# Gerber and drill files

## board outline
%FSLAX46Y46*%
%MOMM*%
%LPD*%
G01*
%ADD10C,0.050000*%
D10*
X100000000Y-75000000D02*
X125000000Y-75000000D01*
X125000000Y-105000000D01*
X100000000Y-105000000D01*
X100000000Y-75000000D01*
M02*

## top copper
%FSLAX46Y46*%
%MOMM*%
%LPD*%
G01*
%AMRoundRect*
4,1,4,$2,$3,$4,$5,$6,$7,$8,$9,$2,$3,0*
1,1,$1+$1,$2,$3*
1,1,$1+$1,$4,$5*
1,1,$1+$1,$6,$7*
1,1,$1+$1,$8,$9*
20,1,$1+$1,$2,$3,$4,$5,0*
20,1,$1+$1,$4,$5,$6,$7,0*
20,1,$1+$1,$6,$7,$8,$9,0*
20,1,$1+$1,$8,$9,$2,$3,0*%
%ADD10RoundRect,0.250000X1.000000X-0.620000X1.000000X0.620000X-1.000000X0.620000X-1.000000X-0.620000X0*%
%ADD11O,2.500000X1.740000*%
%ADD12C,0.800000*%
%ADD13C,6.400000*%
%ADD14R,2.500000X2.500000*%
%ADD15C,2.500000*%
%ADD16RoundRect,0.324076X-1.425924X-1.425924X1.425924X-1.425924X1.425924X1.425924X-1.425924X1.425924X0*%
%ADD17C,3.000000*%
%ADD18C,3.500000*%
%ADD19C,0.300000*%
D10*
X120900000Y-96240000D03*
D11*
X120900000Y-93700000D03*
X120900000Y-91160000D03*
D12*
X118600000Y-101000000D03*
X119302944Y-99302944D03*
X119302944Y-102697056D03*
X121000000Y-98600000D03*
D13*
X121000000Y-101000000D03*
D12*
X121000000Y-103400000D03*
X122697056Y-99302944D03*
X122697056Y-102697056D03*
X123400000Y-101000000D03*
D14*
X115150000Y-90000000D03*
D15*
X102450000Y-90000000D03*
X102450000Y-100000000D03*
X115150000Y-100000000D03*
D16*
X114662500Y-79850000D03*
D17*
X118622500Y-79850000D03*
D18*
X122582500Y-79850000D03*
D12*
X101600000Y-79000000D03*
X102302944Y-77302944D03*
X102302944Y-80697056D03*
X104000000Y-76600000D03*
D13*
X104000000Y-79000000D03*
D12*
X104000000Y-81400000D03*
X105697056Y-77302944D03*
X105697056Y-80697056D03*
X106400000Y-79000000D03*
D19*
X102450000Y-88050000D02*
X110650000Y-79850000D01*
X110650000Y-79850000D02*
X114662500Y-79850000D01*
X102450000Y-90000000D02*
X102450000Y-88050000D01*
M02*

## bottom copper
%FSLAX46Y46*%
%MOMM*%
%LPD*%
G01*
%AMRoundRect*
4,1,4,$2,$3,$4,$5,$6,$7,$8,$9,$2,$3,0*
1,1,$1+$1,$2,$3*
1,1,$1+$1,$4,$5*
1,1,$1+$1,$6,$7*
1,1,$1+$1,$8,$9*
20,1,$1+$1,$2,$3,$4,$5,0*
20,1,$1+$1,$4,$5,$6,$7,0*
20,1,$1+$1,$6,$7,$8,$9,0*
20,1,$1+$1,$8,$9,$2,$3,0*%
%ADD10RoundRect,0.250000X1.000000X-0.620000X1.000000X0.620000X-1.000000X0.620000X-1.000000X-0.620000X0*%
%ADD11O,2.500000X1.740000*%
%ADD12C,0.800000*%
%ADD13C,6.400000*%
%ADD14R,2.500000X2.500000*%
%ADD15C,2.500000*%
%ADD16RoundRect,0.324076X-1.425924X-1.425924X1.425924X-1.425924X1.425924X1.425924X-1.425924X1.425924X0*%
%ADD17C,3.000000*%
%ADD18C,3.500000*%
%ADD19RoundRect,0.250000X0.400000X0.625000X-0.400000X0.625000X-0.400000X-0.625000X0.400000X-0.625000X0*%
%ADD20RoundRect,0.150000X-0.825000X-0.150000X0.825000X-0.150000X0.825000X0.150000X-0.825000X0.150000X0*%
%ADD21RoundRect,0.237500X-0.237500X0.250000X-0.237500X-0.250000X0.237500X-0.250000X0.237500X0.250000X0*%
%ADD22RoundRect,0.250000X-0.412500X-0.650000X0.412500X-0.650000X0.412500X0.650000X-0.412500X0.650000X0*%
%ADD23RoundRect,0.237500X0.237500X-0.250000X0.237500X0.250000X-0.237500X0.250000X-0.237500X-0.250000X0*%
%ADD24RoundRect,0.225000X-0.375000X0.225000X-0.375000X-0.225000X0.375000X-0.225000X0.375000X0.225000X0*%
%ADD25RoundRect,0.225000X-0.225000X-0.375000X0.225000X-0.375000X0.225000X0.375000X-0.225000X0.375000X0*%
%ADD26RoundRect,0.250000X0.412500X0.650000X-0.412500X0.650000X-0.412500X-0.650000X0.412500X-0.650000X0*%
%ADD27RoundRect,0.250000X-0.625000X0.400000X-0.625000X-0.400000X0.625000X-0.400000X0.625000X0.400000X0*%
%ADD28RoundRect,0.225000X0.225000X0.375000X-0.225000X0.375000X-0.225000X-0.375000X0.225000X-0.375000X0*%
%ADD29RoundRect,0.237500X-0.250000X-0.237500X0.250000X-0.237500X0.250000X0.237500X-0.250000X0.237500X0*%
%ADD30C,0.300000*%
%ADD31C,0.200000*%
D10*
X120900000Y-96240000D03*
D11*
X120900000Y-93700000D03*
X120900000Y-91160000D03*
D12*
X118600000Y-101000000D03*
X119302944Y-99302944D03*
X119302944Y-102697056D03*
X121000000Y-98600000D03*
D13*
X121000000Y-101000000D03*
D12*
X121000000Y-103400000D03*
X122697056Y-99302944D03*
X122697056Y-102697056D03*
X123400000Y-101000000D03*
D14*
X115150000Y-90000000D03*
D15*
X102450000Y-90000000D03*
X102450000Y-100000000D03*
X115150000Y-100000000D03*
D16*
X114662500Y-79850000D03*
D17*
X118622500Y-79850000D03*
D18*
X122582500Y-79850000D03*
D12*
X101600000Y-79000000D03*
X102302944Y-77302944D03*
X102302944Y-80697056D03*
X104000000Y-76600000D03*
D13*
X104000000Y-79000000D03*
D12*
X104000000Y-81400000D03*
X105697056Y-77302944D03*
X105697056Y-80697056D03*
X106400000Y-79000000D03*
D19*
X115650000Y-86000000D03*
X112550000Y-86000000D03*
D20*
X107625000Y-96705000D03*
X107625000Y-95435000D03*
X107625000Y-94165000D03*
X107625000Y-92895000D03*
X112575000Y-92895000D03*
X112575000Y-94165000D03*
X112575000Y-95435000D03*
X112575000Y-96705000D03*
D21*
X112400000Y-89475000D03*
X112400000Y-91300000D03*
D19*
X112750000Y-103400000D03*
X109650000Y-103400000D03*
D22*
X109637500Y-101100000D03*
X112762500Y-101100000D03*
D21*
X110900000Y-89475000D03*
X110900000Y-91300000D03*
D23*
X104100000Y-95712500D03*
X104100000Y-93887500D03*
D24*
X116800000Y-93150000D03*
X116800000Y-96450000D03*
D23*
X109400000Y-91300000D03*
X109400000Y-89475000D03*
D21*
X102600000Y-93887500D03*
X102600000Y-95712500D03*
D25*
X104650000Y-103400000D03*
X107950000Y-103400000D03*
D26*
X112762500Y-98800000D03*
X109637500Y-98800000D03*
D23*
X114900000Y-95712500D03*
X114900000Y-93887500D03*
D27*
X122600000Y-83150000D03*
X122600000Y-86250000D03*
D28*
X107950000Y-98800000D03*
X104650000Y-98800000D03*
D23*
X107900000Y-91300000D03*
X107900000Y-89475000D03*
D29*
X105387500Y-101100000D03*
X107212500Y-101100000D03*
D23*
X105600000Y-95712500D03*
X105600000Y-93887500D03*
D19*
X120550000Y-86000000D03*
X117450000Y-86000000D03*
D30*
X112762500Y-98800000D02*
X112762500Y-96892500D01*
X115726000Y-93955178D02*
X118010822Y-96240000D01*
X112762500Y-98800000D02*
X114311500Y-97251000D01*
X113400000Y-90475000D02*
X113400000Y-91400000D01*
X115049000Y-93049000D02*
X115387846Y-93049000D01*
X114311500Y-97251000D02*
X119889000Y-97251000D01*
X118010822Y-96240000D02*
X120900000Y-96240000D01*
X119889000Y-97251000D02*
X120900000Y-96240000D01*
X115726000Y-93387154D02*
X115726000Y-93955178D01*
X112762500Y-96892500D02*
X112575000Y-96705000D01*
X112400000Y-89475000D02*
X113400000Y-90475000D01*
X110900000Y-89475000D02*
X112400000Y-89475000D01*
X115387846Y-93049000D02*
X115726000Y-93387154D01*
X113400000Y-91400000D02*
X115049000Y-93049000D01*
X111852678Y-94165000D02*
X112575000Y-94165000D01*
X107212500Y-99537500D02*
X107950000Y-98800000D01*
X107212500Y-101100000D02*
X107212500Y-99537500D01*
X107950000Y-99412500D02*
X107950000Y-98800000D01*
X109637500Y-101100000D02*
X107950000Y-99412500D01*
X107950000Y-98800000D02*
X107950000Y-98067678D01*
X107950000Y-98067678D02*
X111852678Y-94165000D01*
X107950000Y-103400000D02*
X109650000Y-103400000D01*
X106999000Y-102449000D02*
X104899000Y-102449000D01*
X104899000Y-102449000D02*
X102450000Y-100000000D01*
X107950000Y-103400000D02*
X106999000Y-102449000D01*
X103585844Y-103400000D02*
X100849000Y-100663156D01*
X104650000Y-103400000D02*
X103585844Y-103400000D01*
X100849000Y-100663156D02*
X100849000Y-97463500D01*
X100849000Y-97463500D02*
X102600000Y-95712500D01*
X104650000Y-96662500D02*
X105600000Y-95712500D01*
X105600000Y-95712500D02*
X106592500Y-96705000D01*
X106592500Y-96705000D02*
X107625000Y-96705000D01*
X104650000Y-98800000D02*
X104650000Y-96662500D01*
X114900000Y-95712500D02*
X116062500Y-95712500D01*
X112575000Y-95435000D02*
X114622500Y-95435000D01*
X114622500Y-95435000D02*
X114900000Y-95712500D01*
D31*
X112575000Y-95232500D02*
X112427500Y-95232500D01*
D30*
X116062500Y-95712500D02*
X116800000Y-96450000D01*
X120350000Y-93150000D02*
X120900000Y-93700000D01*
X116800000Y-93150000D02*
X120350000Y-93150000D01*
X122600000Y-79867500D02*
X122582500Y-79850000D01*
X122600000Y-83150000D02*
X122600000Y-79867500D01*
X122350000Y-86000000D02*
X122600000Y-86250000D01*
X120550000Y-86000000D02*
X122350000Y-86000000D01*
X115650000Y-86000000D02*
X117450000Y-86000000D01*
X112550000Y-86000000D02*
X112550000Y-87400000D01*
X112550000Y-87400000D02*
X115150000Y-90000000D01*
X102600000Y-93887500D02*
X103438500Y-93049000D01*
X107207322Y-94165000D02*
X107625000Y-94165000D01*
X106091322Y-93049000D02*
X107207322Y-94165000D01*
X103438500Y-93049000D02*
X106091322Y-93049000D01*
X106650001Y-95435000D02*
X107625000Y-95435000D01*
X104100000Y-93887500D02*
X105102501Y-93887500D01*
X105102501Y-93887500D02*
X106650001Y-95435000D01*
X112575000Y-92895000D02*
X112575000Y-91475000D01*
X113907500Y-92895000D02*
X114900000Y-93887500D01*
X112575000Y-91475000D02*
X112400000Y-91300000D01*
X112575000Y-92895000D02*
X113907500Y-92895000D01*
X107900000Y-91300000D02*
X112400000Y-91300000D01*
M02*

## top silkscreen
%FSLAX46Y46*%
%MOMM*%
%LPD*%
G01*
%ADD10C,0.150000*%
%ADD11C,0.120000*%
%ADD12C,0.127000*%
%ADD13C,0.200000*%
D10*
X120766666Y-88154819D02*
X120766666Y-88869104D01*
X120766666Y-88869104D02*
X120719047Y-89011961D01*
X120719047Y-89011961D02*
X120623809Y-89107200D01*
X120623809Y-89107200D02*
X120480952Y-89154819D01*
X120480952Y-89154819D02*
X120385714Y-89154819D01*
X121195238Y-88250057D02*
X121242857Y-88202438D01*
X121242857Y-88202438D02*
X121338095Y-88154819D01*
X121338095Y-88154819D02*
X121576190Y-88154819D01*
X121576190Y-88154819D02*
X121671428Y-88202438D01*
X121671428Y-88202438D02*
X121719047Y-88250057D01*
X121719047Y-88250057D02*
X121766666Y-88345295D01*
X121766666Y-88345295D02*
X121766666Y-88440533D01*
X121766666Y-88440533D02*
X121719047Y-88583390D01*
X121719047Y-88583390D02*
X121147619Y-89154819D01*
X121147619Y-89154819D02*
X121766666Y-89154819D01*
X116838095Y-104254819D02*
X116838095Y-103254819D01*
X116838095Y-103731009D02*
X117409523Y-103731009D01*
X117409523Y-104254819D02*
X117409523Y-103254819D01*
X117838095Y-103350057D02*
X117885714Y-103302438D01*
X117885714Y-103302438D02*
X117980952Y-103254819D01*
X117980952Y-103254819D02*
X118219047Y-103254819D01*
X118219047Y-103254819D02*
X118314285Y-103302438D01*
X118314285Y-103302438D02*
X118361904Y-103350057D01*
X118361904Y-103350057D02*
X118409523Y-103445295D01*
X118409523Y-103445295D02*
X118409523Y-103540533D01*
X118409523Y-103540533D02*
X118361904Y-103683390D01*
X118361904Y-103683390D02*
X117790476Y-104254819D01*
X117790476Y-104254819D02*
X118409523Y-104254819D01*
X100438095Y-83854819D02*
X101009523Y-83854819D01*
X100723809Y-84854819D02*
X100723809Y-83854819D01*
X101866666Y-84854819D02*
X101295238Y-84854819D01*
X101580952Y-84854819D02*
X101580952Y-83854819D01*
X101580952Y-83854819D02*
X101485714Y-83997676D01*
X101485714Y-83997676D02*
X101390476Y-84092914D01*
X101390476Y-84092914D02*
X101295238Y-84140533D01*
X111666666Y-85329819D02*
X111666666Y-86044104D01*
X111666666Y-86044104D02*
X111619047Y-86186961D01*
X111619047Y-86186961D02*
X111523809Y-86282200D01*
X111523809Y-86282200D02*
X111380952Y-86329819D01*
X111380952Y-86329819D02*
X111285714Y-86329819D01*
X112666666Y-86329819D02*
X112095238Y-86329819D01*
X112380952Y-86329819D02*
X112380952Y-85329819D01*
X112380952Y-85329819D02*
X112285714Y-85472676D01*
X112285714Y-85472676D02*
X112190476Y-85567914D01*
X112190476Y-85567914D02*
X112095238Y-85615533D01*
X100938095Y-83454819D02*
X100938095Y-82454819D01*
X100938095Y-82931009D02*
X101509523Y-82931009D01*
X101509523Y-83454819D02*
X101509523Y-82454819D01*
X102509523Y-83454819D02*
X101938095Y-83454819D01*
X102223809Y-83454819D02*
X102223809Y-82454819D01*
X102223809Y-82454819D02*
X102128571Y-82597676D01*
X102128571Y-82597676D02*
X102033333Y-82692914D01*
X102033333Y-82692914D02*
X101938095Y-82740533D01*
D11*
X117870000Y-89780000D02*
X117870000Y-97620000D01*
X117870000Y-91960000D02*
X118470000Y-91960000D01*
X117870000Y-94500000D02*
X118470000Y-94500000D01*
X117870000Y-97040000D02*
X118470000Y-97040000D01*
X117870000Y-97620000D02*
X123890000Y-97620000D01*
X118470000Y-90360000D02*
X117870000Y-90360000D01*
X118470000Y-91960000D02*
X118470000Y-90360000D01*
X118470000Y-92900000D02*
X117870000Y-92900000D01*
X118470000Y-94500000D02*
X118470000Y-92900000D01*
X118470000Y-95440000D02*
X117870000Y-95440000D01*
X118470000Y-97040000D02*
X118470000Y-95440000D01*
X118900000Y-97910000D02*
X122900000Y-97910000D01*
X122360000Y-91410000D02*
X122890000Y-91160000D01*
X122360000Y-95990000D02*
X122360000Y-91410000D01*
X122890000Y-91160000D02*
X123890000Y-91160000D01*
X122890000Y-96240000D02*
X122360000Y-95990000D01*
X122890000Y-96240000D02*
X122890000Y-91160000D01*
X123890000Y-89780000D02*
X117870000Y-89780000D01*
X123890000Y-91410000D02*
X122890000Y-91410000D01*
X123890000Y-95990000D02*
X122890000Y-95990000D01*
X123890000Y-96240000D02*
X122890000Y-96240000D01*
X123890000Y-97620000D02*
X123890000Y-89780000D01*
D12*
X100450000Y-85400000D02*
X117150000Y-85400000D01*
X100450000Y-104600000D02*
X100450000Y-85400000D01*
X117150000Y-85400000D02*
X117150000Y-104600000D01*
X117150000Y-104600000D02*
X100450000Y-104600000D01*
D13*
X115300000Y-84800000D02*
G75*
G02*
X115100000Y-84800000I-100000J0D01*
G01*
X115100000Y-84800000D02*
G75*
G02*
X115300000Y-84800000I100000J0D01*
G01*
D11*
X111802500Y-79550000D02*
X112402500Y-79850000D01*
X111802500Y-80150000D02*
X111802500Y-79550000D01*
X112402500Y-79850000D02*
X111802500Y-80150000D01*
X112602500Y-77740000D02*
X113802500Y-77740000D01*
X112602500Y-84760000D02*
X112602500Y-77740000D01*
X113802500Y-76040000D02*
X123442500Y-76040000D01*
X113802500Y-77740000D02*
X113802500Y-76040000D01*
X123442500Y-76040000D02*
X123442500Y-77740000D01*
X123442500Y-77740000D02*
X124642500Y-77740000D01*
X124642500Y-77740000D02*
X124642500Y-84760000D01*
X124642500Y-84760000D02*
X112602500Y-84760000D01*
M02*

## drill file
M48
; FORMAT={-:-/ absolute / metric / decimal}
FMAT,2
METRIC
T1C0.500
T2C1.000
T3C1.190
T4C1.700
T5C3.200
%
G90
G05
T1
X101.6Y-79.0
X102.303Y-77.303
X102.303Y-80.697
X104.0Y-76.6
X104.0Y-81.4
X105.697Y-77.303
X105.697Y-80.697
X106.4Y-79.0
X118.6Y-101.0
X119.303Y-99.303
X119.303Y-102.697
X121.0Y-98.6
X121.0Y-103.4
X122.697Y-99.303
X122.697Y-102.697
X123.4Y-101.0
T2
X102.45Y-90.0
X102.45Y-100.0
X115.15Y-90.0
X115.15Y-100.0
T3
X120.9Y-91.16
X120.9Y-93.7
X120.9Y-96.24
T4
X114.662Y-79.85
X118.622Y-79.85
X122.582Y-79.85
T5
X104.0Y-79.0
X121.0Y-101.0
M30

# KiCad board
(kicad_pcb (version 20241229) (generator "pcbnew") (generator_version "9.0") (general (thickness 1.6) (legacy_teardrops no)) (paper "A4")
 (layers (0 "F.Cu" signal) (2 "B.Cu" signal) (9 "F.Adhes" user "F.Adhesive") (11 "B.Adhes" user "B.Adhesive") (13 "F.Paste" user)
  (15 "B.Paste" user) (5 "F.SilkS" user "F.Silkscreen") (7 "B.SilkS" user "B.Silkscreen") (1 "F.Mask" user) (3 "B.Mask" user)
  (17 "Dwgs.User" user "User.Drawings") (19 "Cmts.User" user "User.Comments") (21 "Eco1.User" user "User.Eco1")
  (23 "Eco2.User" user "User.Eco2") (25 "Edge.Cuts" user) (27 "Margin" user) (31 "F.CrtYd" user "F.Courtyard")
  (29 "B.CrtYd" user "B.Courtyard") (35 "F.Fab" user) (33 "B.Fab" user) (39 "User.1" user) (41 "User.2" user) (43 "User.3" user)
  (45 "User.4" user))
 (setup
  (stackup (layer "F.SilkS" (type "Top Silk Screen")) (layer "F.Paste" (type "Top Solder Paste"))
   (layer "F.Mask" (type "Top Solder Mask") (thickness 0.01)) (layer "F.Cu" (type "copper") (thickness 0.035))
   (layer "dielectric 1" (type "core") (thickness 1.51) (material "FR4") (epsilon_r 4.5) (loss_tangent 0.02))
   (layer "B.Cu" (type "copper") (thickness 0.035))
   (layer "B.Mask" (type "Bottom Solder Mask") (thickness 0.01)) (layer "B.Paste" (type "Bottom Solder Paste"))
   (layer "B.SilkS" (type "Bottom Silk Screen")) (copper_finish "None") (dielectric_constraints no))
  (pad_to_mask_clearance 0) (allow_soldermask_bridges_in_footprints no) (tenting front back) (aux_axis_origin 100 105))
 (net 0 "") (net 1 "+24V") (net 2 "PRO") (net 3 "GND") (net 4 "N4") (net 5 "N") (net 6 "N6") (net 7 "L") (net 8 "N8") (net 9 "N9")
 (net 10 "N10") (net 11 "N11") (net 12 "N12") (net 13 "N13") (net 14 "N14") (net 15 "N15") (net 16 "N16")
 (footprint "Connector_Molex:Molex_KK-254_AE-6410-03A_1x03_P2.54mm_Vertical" (layer "F.Cu") (at 120.9 96.24 90)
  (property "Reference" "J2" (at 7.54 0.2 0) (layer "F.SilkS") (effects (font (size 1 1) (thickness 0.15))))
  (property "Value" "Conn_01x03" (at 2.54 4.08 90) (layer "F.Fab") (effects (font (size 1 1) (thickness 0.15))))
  (fp_line (start 6.46 -3.03) (end -1.38 -3.03) (stroke (width 0.12) (type solid)) (layer "F.SilkS"))
  (fp_line (start 4.28 -3.03) (end 4.28 -2.43) (stroke (width 0.12) (type solid)) (layer "F.SilkS"))
  (fp_line (start 1.74 -3.03) (end 1.74 -2.43) (stroke (width 0.12) (type solid)) (layer "F.SilkS"))
  (fp_line (start -0.8 -3.03) (end -0.8 -2.43) (stroke (width 0.12) (type solid)) (layer "F.SilkS"))
  (fp_line (start -1.38 -3.03) (end -1.38 2.99) (stroke (width 0.12) (type solid)) (layer "F.SilkS"))
  (fp_line (start 5.88 -2.43) (end 5.88 -3.03) (stroke (width 0.12) (type solid)) (layer "F.SilkS"))
  (fp_line (start 4.28 -2.43) (end 5.88 -2.43) (stroke (width 0.12) (type solid)) (layer "F.SilkS"))
  (fp_line (start 3.34 -2.43) (end 3.34 -3.03) (stroke (width 0.12) (type solid)) (layer "F.SilkS"))
  (fp_line (start 1.74 -2.43) (end 3.34 -2.43) (stroke (width 0.12) (type solid)) (layer "F.SilkS"))
  (fp_line (start 0.8 -2.43) (end 0.8 -3.03) (stroke (width 0.12) (type solid)) (layer "F.SilkS"))
  (fp_line (start -0.8 -2.43) (end 0.8 -2.43) (stroke (width 0.12) (type solid)) (layer "F.SilkS"))
  (fp_line (start -1.67 -2) (end -1.67 2) (stroke (width 0.12) (type solid)) (layer "F.SilkS"))
  (fp_line (start 4.83 1.46) (end 5.08 1.99) (stroke (width 0.12) (type solid)) (layer "F.SilkS"))
  (fp_line (start 0.25 1.46) (end 4.83 1.46) (stroke (width 0.12) (type solid)) (layer "F.SilkS"))
  (fp_line (start 5.08 1.99) (end 5.08 2.99) (stroke (width 0.12) (type solid)) (layer "F.SilkS"))
  (fp_line (start 0 1.99) (end 0.25 1.46) (stroke (width 0.12) (type solid)) (layer "F.SilkS"))
  (fp_line (start 0 1.99) (end 5.08 1.99) (stroke (width 0.12) (type solid)) (layer "F.SilkS"))
  (fp_line (start 6.46 2.99) (end 6.46 -3.03) (stroke (width 0.12) (type solid)) (layer "F.SilkS"))
  (fp_line (start 4.83 2.99) (end 4.83 1.99) (stroke (width 0.12) (type solid)) (layer "F.SilkS"))
  (fp_line (start 0.25 2.99) (end 0.25 1.99) (stroke (width 0.12) (type solid)) (layer "F.SilkS"))
  (fp_line (start 0 2.99) (end 0 1.99) (stroke (width 0.12) (type solid)) (layer "F.SilkS"))
  (fp_line (start -1.38 2.99) (end 6.46 2.99) (stroke (width 0.12) (type solid)) (layer "F.SilkS"))
  (pad "1" thru_hole roundrect (at 0 0 90) (size 1.74 2.5) (drill 1.19) (layers "*.Cu" "*.Mask") (remove_unused_layers no)
   (roundrect_rratio 0.143678) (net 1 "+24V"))
  (pad "2" thru_hole oval (at 2.54 0 90) (size 1.74 2.5) (drill 1.19) (layers "*.Cu" "*.Mask") (remove_unused_layers no) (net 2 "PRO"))
  (pad "3" thru_hole oval (at 5.08 0 90) (size 1.74 2.5) (drill 1.19) (layers "*.Cu" "*.Mask") (remove_unused_layers no) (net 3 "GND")))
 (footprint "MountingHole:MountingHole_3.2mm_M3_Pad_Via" (layer "F.Cu") (at 121 101)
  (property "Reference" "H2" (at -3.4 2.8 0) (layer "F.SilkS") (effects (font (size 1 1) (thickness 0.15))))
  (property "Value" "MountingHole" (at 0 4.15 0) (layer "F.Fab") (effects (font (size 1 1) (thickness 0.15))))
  (pad "1" thru_hole circle (at -2.4 0) (size 0.8 0.8) (drill 0.5) (layers "*.Cu" "*.Mask") (remove_unused_layers no) (zone_connect 2))
  (pad "1" thru_hole circle (at -1.697056 -1.697056) (size 0.8 0.8) (drill 0.5) (layers "*.Cu" "*.Mask") (remove_unused_layers no)
   (zone_connect 2))
  (pad "1" thru_hole circle (at -1.697056 1.697056) (size 0.8 0.8) (drill 0.5) (layers "*.Cu" "*.Mask") (remove_unused_layers no)
   (zone_connect 2))
  (pad "1" thru_hole circle (at 0 -2.4) (size 0.8 0.8) (drill 0.5) (layers "*.Cu" "*.Mask") (remove_unused_layers no) (zone_connect 2))
  (pad "1" thru_hole circle (at 0 0) (size 6.4 6.4) (drill 3.2) (layers "*.Cu" "*.Mask") (remove_unused_layers no) (zone_connect 2))
  (pad "1" thru_hole circle (at 0 2.4) (size 0.8 0.8) (drill 0.5) (layers "*.Cu" "*.Mask") (remove_unused_layers no) (zone_connect 2))
  (pad "1" thru_hole circle (at 1.697056 -1.697056) (size 0.8 0.8) (drill 0.5) (layers "*.Cu" "*.Mask") (remove_unused_layers no)
   (zone_connect 2))
  (pad "1" thru_hole circle (at 1.697056 1.697056) (size 0.8 0.8) (drill 0.5) (layers "*.Cu" "*.Mask") (remove_unused_layers no)
   (zone_connect 2))
  (pad "1" thru_hole circle (at 2.4 0) (size 0.8 0.8) (drill 0.5) (layers "*.Cu" "*.Mask") (remove_unused_layers no) (zone_connect 2)))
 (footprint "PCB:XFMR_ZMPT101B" (layer "F.Cu") (at 108.8 95 -90)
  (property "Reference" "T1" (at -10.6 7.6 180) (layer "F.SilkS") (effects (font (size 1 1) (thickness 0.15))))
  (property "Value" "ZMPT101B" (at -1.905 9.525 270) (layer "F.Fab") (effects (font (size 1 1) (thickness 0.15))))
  (fp_line (start -9.6 8.35) (end -9.6 -8.35) (stroke (width 0.127) (type solid)) (layer "F.SilkS"))
  (fp_line (start 9.6 8.35) (end -9.6 8.35) (stroke (width 0.127) (type solid)) (layer "F.SilkS"))
  (fp_line (start -9.6 -8.35) (end 9.6 -8.35) (stroke (width 0.127) (type solid)) (layer "F.SilkS"))
  (fp_line (start 9.6 -8.35) (end 9.6 8.35) (stroke (width 0.127) (type solid)) (layer "F.SilkS"))
  (fp_circle (center -10.2 -6.4) (end -10.1 -6.4) (stroke (width 0.2) (type solid)) (fill no) (layer "F.SilkS"))
  (pad "1" thru_hole rect (at -5 -6.35 270) (size 2.5 2.5) (drill 1) (layers "*.Cu" "*.Mask") (remove_unused_layers no) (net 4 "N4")
   (solder_mask_margin 0.102))
  (pad "2" thru_hole circle (at -5 6.35 270) (size 2.5 2.5) (drill 1) (layers "*.Cu" "*.Mask") (remove_unused_layers no) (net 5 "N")
   (solder_mask_margin 0.102))
  (pad "3" thru_hole circle (at 5 6.35 270) (size 2.5 2.5) (drill 1) (layers "*.Cu" "*.Mask") (remove_unused_layers no) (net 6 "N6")
   (solder_mask_margin 0.102))
  (pad "4" thru_hole circle (at 5 -6.35 270) (size 2.5 2.5) (drill 1) (layers "*.Cu" "*.Mask") (remove_unused_layers no) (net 3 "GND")
   (solder_mask_margin 0.102)))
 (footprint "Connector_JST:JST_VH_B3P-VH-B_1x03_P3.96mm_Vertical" (layer "F.Cu") (at 114.6625 79.85)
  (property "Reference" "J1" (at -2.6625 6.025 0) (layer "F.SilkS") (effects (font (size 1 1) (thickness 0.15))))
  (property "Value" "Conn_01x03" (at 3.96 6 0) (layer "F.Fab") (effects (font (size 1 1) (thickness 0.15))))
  (fp_line (start -2.86 -0.3) (end -2.26 0) (stroke (width 0.12) (type solid)) (layer "F.SilkS"))
  (fp_line (start -2.86 0.3) (end -2.86 -0.3) (stroke (width 0.12) (type solid)) (layer "F.SilkS"))
  (fp_line (start -2.26 0) (end -2.86 0.3) (stroke (width 0.12) (type solid)) (layer "F.SilkS"))
  (fp_line (start -2.06 -2.11) (end -0.86 -2.11) (stroke (width 0.12) (type solid)) (layer "F.SilkS"))
  (fp_line (start -2.06 4.91) (end -2.06 -2.11) (stroke (width 0.12) (type solid)) (layer "F.SilkS"))
  (fp_line (start -0.86 -3.81) (end 8.78 -3.81) (stroke (width 0.12) (type solid)) (layer "F.SilkS"))
  (fp_line (start -0.86 -2.11) (end -0.86 -3.81) (stroke (width 0.12) (type solid)) (layer "F.SilkS"))
  (fp_line (start 8.78 -3.81) (end 8.78 -2.11) (stroke (width 0.12) (type solid)) (layer "F.SilkS"))
  (fp_line (start 8.78 -2.11) (end 9.98 -2.11) (stroke (width 0.12) (type solid)) (layer "F.SilkS"))
  (fp_line (start 9.98 -2.11) (end 9.98 4.91) (stroke (width 0.12) (type solid)) (layer "F.SilkS"))
  (fp_line (start 9.98 4.91) (end -2.06 4.91) (stroke (width 0.12) (type solid)) (layer "F.SilkS"))
  (pad "1" thru_hole roundrect (at 0 0) (size 3.5 3.5) (drill 1.7) (layers "*.Cu" "*.Mask") (remove_unused_layers no)
   (roundrect_rratio 0.092593) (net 5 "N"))
  (pad "2" thru_hole circle (at 3.96 0) (size 3 3) (drill 1.7) (layers) (remove_unused_layers no))
  (pad "3" thru_hole circle (at 7.92 0) (size 3.5 3.5) (drill 1.7) (layers "*.Cu" "*.Mask") (remove_unused_layers no) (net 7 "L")))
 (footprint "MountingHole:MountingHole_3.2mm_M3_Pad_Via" (layer "F.Cu") (at 104 79)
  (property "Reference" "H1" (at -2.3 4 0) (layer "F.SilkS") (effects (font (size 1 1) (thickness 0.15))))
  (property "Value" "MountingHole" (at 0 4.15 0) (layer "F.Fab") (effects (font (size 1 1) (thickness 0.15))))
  (pad "1" thru_hole circle (at -2.4 0) (size 0.8 0.8) (drill 0.5) (layers "*.Cu" "*.Mask") (remove_unused_layers no) (zone_connect 2))
  (pad "1" thru_hole circle (at -1.697056 -1.697056) (size 0.8 0.8) (drill 0.5) (layers "*.Cu" "*.Mask") (remove_unused_layers no)
   (zone_connect 2))
  (pad "1" thru_hole circle (at -1.697056 1.697056) (size 0.8 0.8) (drill 0.5) (layers "*.Cu" "*.Mask") (remove_unused_layers no)
   (zone_connect 2))
  (pad "1" thru_hole circle (at 0 -2.4) (size 0.8 0.8) (drill 0.5) (layers "*.Cu" "*.Mask") (remove_unused_layers no) (zone_connect 2))
  (pad "1" thru_hole circle (at 0 0) (size 6.4 6.4) (drill 3.2) (layers "*.Cu" "*.Mask") (remove_unused_layers no) (zone_connect 2))
  (pad "1" thru_hole circle (at 0 2.4) (size 0.8 0.8) (drill 0.5) (layers "*.Cu" "*.Mask") (remove_unused_layers no) (zone_connect 2))
  (pad "1" thru_hole circle (at 1.697056 -1.697056) (size 0.8 0.8) (drill 0.5) (layers "*.Cu" "*.Mask") (remove_unused_layers no)
   (zone_connect 2))
  (pad "1" thru_hole circle (at 1.697056 1.697056) (size 0.8 0.8) (drill 0.5) (layers "*.Cu" "*.Mask") (remove_unused_layers no)
   (zone_connect 2))
  (pad "1" thru_hole circle (at 2.4 0) (size 0.8 0.8) (drill 0.5) (layers "*.Cu" "*.Mask") (remove_unused_layers no) (zone_connect 2)))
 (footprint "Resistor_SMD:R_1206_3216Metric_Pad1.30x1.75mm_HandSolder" (layer "B.Cu") (at 114.1 86 180)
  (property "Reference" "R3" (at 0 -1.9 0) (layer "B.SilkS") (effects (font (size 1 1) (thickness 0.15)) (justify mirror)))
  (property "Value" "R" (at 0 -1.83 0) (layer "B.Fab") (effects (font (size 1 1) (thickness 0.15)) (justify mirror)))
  (pad "1" smd roundrect (at -1.55 0 180) (size 1.3 1.75) (layers "B.Cu" "B.Mask" "B.Paste") (roundrect_rratio 0.192308) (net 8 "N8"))
  (pad "2" smd roundrect (at 1.55 0 180) (size 1.3 1.75) (layers "B.Cu" "B.Mask" "B.Paste") (roundrect_rratio 0.192308) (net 4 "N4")))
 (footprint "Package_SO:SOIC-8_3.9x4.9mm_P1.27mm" (layer "B.Cu") (at 110.1 94.8)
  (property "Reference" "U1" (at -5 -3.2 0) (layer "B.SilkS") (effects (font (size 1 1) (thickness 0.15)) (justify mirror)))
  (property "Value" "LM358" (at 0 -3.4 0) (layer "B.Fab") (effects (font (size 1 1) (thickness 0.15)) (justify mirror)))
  (pad "1" smd roundrect (at -2.475 1.905) (size 1.95 0.6) (layers "B.Cu" "B.Mask" "B.Paste") (roundrect_rratio 0.25) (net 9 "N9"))
  (pad "2" smd roundrect (at -2.475 0.635) (size 1.95 0.6) (layers "B.Cu" "B.Mask" "B.Paste") (roundrect_rratio 0.25) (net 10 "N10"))
  (pad "3" smd roundrect (at -2.475 -0.635) (size 1.95 0.6) (layers "B.Cu" "B.Mask" "B.Paste") (roundrect_rratio 0.25) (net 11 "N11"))
  (pad "4" smd roundrect (at -2.475 -1.905) (size 1.95 0.6) (layers "B.Cu" "B.Mask" "B.Paste") (roundrect_rratio 0.25) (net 3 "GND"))
  (pad "5" smd roundrect (at 2.475 -1.905) (size 1.95 0.6) (layers "B.Cu" "B.Mask" "B.Paste") (roundrect_rratio 0.25) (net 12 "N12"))
  (pad "6" smd roundrect (at 2.475 -0.635) (size 1.95 0.6) (layers "B.Cu" "B.Mask" "B.Paste") (roundrect_rratio 0.25) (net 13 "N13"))
  (pad "7" smd roundrect (at 2.475 0.635) (size 1.95 0.6) (layers "B.Cu" "B.Mask" "B.Paste") (roundrect_rratio 0.25) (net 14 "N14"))
  (pad "8" smd roundrect (at 2.475 1.905) (size 1.95 0.6) (layers "B.Cu" "B.Mask" "B.Paste") (roundrect_rratio 0.25) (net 1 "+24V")))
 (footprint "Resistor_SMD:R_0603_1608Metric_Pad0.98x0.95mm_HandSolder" (layer "B.Cu") (at 112.4 90.3875 -90)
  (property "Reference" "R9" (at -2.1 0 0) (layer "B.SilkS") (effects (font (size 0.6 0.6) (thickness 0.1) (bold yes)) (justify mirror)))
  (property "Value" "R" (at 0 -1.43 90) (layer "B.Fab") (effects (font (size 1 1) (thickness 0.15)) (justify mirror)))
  (pad "1" smd roundrect (at -0.9125 0 270) (size 0.975 0.95) (layers "B.Cu" "B.Mask" "B.Paste") (roundrect_rratio 0.25) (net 1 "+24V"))
  (pad "2" smd roundrect (at 0.9125 0 270) (size 0.975 0.95) (layers "B.Cu" "B.Mask" "B.Paste") (roundrect_rratio 0.25) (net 12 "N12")))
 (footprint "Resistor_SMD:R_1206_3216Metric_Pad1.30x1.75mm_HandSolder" (layer "B.Cu") (at 111.2 103.4 180)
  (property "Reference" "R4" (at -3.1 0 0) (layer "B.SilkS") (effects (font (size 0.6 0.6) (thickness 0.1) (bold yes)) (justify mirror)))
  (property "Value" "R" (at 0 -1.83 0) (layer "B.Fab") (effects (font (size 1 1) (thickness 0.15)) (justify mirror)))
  (pad "1" smd roundrect (at -1.55 0 180) (size 1.3 1.75) (layers "B.Cu" "B.Mask" "B.Paste") (roundrect_rratio 0.192308) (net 3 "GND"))
  (pad "2" smd roundrect (at 1.55 0 180) (size 1.3 1.75) (layers "B.Cu" "B.Mask" "B.Paste") (roundrect_rratio 0.192308) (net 6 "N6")))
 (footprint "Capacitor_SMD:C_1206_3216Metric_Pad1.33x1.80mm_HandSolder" (layer "B.Cu") (at 111.2 101.1)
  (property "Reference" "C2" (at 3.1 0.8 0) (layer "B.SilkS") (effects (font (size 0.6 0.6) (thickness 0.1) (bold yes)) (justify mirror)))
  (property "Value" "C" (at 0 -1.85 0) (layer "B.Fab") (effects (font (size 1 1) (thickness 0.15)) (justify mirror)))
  (pad "1" smd roundrect (at -1.5625 0) (size 1.325 1.8) (layers "B.Cu" "B.Mask" "B.Paste") (roundrect_rratio 0.188679) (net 13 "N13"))
  (pad "2" smd roundrect (at 1.5625 0) (size 1.325 1.8) (layers "B.Cu" "B.Mask" "B.Paste") (roundrect_rratio 0.188679) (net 3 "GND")))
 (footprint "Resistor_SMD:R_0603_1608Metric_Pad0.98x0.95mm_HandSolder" (layer "B.Cu") (at 110.9 90.3875 -90)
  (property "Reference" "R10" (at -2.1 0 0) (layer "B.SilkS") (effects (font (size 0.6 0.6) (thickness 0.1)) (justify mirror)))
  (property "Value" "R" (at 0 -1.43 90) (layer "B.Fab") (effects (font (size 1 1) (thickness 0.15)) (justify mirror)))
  (pad "1" smd roundrect (at -0.9125 0 270) (size 0.975 0.95) (layers "B.Cu" "B.Mask" "B.Paste") (roundrect_rratio 0.25) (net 1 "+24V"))
  (pad "2" smd roundrect (at 0.9125 0 270) (size 0.975 0.95) (layers "B.Cu" "B.Mask" "B.Paste") (roundrect_rratio 0.25) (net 12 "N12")))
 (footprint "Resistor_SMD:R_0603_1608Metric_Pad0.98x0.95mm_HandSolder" (layer "B.Cu") (at 104.1 94.8 90)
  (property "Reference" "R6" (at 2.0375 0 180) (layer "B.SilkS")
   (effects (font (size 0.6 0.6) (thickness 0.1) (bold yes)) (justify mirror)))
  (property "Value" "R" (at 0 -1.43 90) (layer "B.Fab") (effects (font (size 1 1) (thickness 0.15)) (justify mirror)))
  (pad "1" smd roundrect (at -0.9125 0 90) (size 0.975 0.95) (layers "B.Cu" "B.Mask" "B.Paste") (roundrect_rratio 0.25) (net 3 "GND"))
  (pad "2" smd roundrect (at 0.9125 0 90) (size 0.975 0.95) (layers "B.Cu" "B.Mask" "B.Paste") (roundrect_rratio 0.25) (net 10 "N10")))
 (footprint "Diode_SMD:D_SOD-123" (layer "B.Cu") (at 116.8 94.8 -90)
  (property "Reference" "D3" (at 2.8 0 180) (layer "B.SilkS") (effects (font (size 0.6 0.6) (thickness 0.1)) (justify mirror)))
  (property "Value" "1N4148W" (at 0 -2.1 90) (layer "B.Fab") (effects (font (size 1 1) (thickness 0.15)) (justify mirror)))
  (pad "1" smd roundrect (at -1.65 0 270) (size 0.9 1.2) (layers "B.Cu" "B.Mask" "B.Paste") (roundrect_rratio 0.25) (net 2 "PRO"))
  (pad "2" smd roundrect (at 1.65 0 270) (size 0.9 1.2) (layers "B.Cu" "B.Mask" "B.Paste") (roundrect_rratio 0.25) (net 14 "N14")))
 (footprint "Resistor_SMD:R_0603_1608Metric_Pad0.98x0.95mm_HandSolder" (layer "B.Cu") (at 109.4 90.3875 90)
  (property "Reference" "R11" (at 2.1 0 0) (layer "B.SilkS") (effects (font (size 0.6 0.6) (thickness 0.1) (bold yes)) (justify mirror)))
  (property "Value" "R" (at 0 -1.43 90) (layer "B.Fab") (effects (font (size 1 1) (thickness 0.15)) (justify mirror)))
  (pad "1" smd roundrect (at -0.9125 0 90) (size 0.975 0.95) (layers "B.Cu" "B.Mask" "B.Paste") (roundrect_rratio 0.25) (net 12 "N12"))
  (pad "2" smd roundrect (at 0.9125 0 90) (size 0.975 0.95) (layers "B.Cu" "B.Mask" "B.Paste") (roundrect_rratio 0.25) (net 3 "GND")))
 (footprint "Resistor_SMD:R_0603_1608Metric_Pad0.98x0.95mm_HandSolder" (layer "B.Cu") (at 102.6 94.8 -90)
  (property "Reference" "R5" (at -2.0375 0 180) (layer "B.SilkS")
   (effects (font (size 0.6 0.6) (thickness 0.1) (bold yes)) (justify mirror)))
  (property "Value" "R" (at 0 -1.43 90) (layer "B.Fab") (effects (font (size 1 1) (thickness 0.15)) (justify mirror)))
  (pad "1" smd roundrect (at -0.9125 0 270) (size 0.975 0.95) (layers "B.Cu" "B.Mask" "B.Paste") (roundrect_rratio 0.25) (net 11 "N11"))
  (pad "2" smd roundrect (at 0.9125 0 270) (size 0.975 0.95) (layers "B.Cu" "B.Mask" "B.Paste") (roundrect_rratio 0.25) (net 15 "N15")))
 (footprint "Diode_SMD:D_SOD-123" (layer "B.Cu") (at 106.3 103.4)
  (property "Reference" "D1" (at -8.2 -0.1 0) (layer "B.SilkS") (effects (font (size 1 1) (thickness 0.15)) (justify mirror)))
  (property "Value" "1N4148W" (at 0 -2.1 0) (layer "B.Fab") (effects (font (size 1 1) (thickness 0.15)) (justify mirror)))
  (pad "1" smd roundrect (at -1.65 0) (size 0.9 1.2) (layers "B.Cu" "B.Mask" "B.Paste") (roundrect_rratio 0.25) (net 15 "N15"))
  (pad "2" smd roundrect (at 1.65 0) (size 0.9 1.2) (layers "B.Cu" "B.Mask" "B.Paste") (roundrect_rratio 0.25) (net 6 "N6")))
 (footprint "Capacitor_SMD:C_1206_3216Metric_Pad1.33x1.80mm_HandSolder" (layer "B.Cu") (at 111.2 98.8 180)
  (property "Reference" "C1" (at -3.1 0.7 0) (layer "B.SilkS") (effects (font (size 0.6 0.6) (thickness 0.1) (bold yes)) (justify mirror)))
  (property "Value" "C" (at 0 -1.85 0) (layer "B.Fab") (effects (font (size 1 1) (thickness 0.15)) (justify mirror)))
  (pad "1" smd roundrect (at -1.5625 0 180) (size 1.325 1.8) (layers "B.Cu" "B.Mask" "B.Paste") (roundrect_rratio 0.188679) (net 1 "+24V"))
  (pad "2" smd roundrect (at 1.5625 0 180) (size 1.325 1.8) (layers "B.Cu" "B.Mask" "B.Paste") (roundrect_rratio 0.188679) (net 3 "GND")))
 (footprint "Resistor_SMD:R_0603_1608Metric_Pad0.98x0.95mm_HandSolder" (layer "B.Cu") (at 114.9 94.8 90)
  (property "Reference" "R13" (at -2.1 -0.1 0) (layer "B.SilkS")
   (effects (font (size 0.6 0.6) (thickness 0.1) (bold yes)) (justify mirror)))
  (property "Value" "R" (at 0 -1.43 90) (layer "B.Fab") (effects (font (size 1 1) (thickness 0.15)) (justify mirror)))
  (pad "1" smd roundrect (at -0.9125 0 90) (size 0.975 0.95) (layers "B.Cu" "B.Mask" "B.Paste") (roundrect_rratio 0.25) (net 14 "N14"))
  (pad "2" smd roundrect (at 0.9125 0 90) (size 0.975 0.95) (layers "B.Cu" "B.Mask" "B.Paste") (roundrect_rratio 0.25) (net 12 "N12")))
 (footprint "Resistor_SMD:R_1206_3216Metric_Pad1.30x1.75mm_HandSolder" (layer "B.Cu") (at 122.6 84.7 -90)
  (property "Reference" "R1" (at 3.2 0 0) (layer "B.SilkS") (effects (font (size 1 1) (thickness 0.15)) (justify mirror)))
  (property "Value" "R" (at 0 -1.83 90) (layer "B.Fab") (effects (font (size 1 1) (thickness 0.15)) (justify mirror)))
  (pad "1" smd roundrect (at -1.55 0 270) (size 1.3 1.75) (layers "B.Cu" "B.Mask" "B.Paste") (roundrect_rratio 0.192308) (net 7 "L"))
  (pad "2" smd roundrect (at 1.55 0 270) (size 1.3 1.75) (layers "B.Cu" "B.Mask" "B.Paste") (roundrect_rratio 0.192308) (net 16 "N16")))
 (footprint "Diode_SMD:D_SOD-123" (layer "B.Cu") (at 106.3 98.8 180)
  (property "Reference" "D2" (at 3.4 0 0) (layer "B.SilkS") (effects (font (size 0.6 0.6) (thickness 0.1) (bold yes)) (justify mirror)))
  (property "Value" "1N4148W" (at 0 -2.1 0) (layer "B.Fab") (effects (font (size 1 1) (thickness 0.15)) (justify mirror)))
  (pad "1" smd roundrect (at -1.65 0 180) (size 0.9 1.2) (layers "B.Cu" "B.Mask" "B.Paste") (roundrect_rratio 0.25) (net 13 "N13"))
  (pad "2" smd roundrect (at 1.65 0 180) (size 0.9 1.2) (layers "B.Cu" "B.Mask" "B.Paste") (roundrect_rratio 0.25) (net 9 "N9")))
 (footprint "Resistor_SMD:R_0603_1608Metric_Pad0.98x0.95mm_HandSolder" (layer "B.Cu") (at 107.9 90.3875 90)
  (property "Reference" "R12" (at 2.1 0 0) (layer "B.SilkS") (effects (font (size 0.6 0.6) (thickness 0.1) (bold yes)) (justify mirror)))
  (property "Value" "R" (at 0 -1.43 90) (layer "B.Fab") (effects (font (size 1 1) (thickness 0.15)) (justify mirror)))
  (pad "1" smd roundrect (at -0.9125 0 90) (size 0.975 0.95) (layers "B.Cu" "B.Mask" "B.Paste") (roundrect_rratio 0.25) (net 12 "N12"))
  (pad "2" smd roundrect (at 0.9125 0 90) (size 0.975 0.95) (layers "B.Cu" "B.Mask" "B.Paste") (roundrect_rratio 0.25) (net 3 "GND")))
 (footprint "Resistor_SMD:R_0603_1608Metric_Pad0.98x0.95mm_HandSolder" (layer "B.Cu") (at 106.3 101.1)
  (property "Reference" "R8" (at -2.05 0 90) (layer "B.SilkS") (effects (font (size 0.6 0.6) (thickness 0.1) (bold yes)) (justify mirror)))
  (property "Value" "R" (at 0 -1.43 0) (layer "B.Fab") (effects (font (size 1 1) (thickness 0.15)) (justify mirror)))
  (pad "1" smd roundrect (at -0.9125 0) (size 0.975 0.95) (layers "B.Cu" "B.Mask" "B.Paste") (roundrect_rratio 0.25) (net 3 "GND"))
  (pad "2" smd roundrect (at 0.9125 0) (size 0.975 0.95) (layers "B.Cu" "B.Mask" "B.Paste") (roundrect_rratio 0.25) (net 13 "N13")))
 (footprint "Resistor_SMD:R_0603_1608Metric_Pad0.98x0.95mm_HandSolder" (layer "B.Cu") (at 105.6 94.8 90)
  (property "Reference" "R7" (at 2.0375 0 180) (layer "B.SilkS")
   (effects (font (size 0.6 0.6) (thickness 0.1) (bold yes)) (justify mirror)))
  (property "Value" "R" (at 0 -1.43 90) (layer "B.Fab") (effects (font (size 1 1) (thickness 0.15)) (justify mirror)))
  (pad "1" smd roundrect (at -0.9125 0 90) (size 0.975 0.95) (layers "B.Cu" "B.Mask" "B.Paste") (roundrect_rratio 0.25) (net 9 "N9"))
  (pad "2" smd roundrect (at 0.9125 0 90) (size 0.975 0.95) (layers "B.Cu" "B.Mask" "B.Paste") (roundrect_rratio 0.25) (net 10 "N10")))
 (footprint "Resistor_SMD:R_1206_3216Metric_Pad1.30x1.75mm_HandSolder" (layer "B.Cu") (at 119 86 180)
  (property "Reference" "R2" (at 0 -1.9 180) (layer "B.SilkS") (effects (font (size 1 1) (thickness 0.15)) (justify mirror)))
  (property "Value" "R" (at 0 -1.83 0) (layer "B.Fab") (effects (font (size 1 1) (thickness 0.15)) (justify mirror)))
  (pad "1" smd roundrect (at -1.55 0 180) (size 1.3 1.75) (layers "B.Cu" "B.Mask" "B.Paste") (roundrect_rratio 0.192308) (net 16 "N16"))
  (pad "2" smd roundrect (at 1.55 0 180) (size 1.3 1.75) (layers "B.Cu" "B.Mask" "B.Paste") (roundrect_rratio 0.192308) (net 8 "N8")))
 (gr_rect (start 100 75) (end 125 105) (stroke (width 0.05) (type solid)) (fill no) (layer "Edge.Cuts"))
 (segment (start 112.7625 98.8) (end 112.7625 96.8925) (width 0.3) (layer "B.Cu") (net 1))
 (segment (start 115.726 93.955178) (end 118.010822 96.24) (width 0.3) (layer "B.Cu") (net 1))
 (segment (start 112.7625 98.8) (end 114.3115 97.251) (width 0.3) (layer "B.Cu") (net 1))
 (segment (start 113.4 90.475) (end 113.4 91.4) (width 0.3) (layer "B.Cu") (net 1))
 (segment (start 115.049 93.049) (end 115.387846 93.049) (width 0.3) (layer "B.Cu") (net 1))
 (segment (start 114.3115 97.251) (end 119.889 97.251) (width 0.3) (layer "B.Cu") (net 1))
 (segment (start 118.010822 96.24) (end 120.9 96.24) (width 0.3) (layer "B.Cu") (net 1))
 (segment (start 119.889 97.251) (end 120.9 96.24) (width 0.3) (layer "B.Cu") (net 1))
 (segment (start 115.726 93.387154) (end 115.726 93.955178) (width 0.3) (layer "B.Cu") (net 1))
 (segment (start 112.7625 96.8925) (end 112.575 96.705) (width 0.3) (layer "B.Cu") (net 1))
 (segment (start 112.4 89.475) (end 113.4 90.475) (width 0.3) (layer "B.Cu") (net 1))
 (segment (start 110.9 89.475) (end 112.4 89.475) (width 0.3) (layer "B.Cu") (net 1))
 (segment (start 115.387846 93.049) (end 115.726 93.387154) (width 0.3) (layer "B.Cu") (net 1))
 (segment (start 113.4 91.4) (end 115.049 93.049) (width 0.3) (layer "B.Cu") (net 1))
 (segment (start 111.852678 94.165) (end 112.575 94.165) (width 0.3) (layer "B.Cu") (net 13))
 (segment (start 107.2125 99.5375) (end 107.95 98.8) (width 0.3) (layer "B.Cu") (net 13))
 (segment (start 107.2125 101.1) (end 107.2125 99.5375) (width 0.3) (layer "B.Cu") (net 13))
 (segment (start 107.95 99.4125) (end 107.95 98.8) (width 0.3) (layer "B.Cu") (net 13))
 (segment (start 109.6375 101.1) (end 107.95 99.4125) (width 0.3) (layer "B.Cu") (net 13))
 (segment (start 107.95 98.8) (end 107.95 98.067678) (width 0.3) (layer "B.Cu") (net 13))
 (segment (start 107.95 98.067678) (end 111.852678 94.165) (width 0.3) (layer "B.Cu") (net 13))
 (segment (start 107.95 103.4) (end 109.65 103.4) (width 0.3) (layer "B.Cu") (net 6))
 (segment (start 106.999 102.449) (end 104.899 102.449) (width 0.3) (layer "B.Cu") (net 6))
 (segment (start 104.899 102.449) (end 102.45 100) (width 0.3) (layer "B.Cu") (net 6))
 (segment (start 107.95 103.4) (end 106.999 102.449) (width 0.3) (layer "B.Cu") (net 6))
 (segment (start 103.585844 103.4) (end 100.849 100.663156) (width 0.3) (layer "B.Cu") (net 15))
 (segment (start 104.65 103.4) (end 103.585844 103.4) (width 0.3) (layer "B.Cu") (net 15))
 (segment (start 100.849 100.663156) (end 100.849 97.4635) (width 0.3) (layer "B.Cu") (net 15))
 (segment (start 100.849 97.4635) (end 102.6 95.7125) (width 0.3) (layer "B.Cu") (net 15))
 (segment (start 104.65 96.6625) (end 105.6 95.7125) (width 0.3) (layer "B.Cu") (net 9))
 (segment (start 105.6 95.7125) (end 106.5925 96.705) (width 0.3) (layer "B.Cu") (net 9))
 (segment (start 106.5925 96.705) (end 107.625 96.705) (width 0.3) (layer "B.Cu") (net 9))
 (segment (start 104.65 98.8) (end 104.65 96.6625) (width 0.3) (layer "B.Cu") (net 9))
 (segment (start 114.9 95.7125) (end 116.0625 95.7125) (width 0.3) (layer "B.Cu") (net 14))
 (segment (start 112.575 95.435) (end 114.6225 95.435) (width 0.3) (layer "B.Cu") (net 14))
 (segment (start 114.6225 95.435) (end 114.9 95.7125) (width 0.3) (layer "B.Cu") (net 14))
 (segment (start 112.575 95.2325) (end 112.4275 95.2325) (width 0.2) (layer "B.Cu") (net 14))
 (segment (start 116.0625 95.7125) (end 116.8 96.45) (width 0.3) (layer "B.Cu") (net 14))
 (segment (start 120.35 93.15) (end 120.9 93.7) (width 0.3) (layer "B.Cu") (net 2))
 (segment (start 116.8 93.15) (end 120.35 93.15) (width 0.3) (layer "B.Cu") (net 2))
 (segment (start 102.45 88.05) (end 110.65 79.85) (width 0.3) (layer "F.Cu") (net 5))
 (segment (start 110.65 79.85) (end 114.6625 79.85) (width 0.3) (layer "F.Cu") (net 5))
 (segment (start 102.45 90) (end 102.45 88.05) (width 0.3) (layer "F.Cu") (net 5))
 (segment (start 122.6 79.8675) (end 122.5825 79.85) (width 0.3) (layer "B.Cu") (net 7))
 (segment (start 122.6 83.15) (end 122.6 79.8675) (width 0.3) (layer "B.Cu") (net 7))
 (segment (start 122.35 86) (end 122.6 86.25) (width 0.3) (layer "B.Cu") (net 16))
 (segment (start 120.55 86) (end 122.35 86) (width 0.3) (layer "B.Cu") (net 16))
 (segment (start 115.65 86) (end 117.45 86) (width 0.3) (layer "B.Cu") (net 8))
 (segment (start 112.55 86) (end 112.55 87.4) (width 0.3) (layer "B.Cu") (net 4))
 (segment (start 112.55 87.4) (end 115.15 90) (width 0.3) (layer "B.Cu") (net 4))
 (segment (start 102.6 93.8875) (end 103.4385 93.049) (width 0.3) (layer "B.Cu") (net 11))
 (segment (start 107.207322 94.165) (end 107.625 94.165) (width 0.3) (layer "B.Cu") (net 11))
 (segment (start 106.091322 93.049) (end 107.207322 94.165) (width 0.3) (layer "B.Cu") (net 11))
 (segment (start 103.4385 93.049) (end 106.091322 93.049) (width 0.3) (layer "B.Cu") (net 11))
 (segment (start 106.650001 95.435) (end 107.625 95.435) (width 0.3) (layer "B.Cu") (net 10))
 (segment (start 104.1 93.8875) (end 105.102501 93.8875) (width 0.3) (layer "B.Cu") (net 10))
 (segment (start 105.102501 93.8875) (end 106.650001 95.435) (width 0.3) (layer "B.Cu") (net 10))
 (segment (start 112.575 92.895) (end 112.575 91.475) (width 0.3) (layer "B.Cu") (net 12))
 (segment (start 113.9075 92.895) (end 114.9 93.8875) (width 0.3) (layer "B.Cu") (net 12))
 (segment (start 112.575 91.475) (end 112.4 91.3) (width 0.3) (layer "B.Cu") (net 12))
 (segment (start 112.575 92.895) (end 113.9075 92.895) (width 0.3) (layer "B.Cu") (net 12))
 (segment (start 107.9 91.3) (end 112.4 91.3) (width 0.3) (layer "B.Cu") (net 12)))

